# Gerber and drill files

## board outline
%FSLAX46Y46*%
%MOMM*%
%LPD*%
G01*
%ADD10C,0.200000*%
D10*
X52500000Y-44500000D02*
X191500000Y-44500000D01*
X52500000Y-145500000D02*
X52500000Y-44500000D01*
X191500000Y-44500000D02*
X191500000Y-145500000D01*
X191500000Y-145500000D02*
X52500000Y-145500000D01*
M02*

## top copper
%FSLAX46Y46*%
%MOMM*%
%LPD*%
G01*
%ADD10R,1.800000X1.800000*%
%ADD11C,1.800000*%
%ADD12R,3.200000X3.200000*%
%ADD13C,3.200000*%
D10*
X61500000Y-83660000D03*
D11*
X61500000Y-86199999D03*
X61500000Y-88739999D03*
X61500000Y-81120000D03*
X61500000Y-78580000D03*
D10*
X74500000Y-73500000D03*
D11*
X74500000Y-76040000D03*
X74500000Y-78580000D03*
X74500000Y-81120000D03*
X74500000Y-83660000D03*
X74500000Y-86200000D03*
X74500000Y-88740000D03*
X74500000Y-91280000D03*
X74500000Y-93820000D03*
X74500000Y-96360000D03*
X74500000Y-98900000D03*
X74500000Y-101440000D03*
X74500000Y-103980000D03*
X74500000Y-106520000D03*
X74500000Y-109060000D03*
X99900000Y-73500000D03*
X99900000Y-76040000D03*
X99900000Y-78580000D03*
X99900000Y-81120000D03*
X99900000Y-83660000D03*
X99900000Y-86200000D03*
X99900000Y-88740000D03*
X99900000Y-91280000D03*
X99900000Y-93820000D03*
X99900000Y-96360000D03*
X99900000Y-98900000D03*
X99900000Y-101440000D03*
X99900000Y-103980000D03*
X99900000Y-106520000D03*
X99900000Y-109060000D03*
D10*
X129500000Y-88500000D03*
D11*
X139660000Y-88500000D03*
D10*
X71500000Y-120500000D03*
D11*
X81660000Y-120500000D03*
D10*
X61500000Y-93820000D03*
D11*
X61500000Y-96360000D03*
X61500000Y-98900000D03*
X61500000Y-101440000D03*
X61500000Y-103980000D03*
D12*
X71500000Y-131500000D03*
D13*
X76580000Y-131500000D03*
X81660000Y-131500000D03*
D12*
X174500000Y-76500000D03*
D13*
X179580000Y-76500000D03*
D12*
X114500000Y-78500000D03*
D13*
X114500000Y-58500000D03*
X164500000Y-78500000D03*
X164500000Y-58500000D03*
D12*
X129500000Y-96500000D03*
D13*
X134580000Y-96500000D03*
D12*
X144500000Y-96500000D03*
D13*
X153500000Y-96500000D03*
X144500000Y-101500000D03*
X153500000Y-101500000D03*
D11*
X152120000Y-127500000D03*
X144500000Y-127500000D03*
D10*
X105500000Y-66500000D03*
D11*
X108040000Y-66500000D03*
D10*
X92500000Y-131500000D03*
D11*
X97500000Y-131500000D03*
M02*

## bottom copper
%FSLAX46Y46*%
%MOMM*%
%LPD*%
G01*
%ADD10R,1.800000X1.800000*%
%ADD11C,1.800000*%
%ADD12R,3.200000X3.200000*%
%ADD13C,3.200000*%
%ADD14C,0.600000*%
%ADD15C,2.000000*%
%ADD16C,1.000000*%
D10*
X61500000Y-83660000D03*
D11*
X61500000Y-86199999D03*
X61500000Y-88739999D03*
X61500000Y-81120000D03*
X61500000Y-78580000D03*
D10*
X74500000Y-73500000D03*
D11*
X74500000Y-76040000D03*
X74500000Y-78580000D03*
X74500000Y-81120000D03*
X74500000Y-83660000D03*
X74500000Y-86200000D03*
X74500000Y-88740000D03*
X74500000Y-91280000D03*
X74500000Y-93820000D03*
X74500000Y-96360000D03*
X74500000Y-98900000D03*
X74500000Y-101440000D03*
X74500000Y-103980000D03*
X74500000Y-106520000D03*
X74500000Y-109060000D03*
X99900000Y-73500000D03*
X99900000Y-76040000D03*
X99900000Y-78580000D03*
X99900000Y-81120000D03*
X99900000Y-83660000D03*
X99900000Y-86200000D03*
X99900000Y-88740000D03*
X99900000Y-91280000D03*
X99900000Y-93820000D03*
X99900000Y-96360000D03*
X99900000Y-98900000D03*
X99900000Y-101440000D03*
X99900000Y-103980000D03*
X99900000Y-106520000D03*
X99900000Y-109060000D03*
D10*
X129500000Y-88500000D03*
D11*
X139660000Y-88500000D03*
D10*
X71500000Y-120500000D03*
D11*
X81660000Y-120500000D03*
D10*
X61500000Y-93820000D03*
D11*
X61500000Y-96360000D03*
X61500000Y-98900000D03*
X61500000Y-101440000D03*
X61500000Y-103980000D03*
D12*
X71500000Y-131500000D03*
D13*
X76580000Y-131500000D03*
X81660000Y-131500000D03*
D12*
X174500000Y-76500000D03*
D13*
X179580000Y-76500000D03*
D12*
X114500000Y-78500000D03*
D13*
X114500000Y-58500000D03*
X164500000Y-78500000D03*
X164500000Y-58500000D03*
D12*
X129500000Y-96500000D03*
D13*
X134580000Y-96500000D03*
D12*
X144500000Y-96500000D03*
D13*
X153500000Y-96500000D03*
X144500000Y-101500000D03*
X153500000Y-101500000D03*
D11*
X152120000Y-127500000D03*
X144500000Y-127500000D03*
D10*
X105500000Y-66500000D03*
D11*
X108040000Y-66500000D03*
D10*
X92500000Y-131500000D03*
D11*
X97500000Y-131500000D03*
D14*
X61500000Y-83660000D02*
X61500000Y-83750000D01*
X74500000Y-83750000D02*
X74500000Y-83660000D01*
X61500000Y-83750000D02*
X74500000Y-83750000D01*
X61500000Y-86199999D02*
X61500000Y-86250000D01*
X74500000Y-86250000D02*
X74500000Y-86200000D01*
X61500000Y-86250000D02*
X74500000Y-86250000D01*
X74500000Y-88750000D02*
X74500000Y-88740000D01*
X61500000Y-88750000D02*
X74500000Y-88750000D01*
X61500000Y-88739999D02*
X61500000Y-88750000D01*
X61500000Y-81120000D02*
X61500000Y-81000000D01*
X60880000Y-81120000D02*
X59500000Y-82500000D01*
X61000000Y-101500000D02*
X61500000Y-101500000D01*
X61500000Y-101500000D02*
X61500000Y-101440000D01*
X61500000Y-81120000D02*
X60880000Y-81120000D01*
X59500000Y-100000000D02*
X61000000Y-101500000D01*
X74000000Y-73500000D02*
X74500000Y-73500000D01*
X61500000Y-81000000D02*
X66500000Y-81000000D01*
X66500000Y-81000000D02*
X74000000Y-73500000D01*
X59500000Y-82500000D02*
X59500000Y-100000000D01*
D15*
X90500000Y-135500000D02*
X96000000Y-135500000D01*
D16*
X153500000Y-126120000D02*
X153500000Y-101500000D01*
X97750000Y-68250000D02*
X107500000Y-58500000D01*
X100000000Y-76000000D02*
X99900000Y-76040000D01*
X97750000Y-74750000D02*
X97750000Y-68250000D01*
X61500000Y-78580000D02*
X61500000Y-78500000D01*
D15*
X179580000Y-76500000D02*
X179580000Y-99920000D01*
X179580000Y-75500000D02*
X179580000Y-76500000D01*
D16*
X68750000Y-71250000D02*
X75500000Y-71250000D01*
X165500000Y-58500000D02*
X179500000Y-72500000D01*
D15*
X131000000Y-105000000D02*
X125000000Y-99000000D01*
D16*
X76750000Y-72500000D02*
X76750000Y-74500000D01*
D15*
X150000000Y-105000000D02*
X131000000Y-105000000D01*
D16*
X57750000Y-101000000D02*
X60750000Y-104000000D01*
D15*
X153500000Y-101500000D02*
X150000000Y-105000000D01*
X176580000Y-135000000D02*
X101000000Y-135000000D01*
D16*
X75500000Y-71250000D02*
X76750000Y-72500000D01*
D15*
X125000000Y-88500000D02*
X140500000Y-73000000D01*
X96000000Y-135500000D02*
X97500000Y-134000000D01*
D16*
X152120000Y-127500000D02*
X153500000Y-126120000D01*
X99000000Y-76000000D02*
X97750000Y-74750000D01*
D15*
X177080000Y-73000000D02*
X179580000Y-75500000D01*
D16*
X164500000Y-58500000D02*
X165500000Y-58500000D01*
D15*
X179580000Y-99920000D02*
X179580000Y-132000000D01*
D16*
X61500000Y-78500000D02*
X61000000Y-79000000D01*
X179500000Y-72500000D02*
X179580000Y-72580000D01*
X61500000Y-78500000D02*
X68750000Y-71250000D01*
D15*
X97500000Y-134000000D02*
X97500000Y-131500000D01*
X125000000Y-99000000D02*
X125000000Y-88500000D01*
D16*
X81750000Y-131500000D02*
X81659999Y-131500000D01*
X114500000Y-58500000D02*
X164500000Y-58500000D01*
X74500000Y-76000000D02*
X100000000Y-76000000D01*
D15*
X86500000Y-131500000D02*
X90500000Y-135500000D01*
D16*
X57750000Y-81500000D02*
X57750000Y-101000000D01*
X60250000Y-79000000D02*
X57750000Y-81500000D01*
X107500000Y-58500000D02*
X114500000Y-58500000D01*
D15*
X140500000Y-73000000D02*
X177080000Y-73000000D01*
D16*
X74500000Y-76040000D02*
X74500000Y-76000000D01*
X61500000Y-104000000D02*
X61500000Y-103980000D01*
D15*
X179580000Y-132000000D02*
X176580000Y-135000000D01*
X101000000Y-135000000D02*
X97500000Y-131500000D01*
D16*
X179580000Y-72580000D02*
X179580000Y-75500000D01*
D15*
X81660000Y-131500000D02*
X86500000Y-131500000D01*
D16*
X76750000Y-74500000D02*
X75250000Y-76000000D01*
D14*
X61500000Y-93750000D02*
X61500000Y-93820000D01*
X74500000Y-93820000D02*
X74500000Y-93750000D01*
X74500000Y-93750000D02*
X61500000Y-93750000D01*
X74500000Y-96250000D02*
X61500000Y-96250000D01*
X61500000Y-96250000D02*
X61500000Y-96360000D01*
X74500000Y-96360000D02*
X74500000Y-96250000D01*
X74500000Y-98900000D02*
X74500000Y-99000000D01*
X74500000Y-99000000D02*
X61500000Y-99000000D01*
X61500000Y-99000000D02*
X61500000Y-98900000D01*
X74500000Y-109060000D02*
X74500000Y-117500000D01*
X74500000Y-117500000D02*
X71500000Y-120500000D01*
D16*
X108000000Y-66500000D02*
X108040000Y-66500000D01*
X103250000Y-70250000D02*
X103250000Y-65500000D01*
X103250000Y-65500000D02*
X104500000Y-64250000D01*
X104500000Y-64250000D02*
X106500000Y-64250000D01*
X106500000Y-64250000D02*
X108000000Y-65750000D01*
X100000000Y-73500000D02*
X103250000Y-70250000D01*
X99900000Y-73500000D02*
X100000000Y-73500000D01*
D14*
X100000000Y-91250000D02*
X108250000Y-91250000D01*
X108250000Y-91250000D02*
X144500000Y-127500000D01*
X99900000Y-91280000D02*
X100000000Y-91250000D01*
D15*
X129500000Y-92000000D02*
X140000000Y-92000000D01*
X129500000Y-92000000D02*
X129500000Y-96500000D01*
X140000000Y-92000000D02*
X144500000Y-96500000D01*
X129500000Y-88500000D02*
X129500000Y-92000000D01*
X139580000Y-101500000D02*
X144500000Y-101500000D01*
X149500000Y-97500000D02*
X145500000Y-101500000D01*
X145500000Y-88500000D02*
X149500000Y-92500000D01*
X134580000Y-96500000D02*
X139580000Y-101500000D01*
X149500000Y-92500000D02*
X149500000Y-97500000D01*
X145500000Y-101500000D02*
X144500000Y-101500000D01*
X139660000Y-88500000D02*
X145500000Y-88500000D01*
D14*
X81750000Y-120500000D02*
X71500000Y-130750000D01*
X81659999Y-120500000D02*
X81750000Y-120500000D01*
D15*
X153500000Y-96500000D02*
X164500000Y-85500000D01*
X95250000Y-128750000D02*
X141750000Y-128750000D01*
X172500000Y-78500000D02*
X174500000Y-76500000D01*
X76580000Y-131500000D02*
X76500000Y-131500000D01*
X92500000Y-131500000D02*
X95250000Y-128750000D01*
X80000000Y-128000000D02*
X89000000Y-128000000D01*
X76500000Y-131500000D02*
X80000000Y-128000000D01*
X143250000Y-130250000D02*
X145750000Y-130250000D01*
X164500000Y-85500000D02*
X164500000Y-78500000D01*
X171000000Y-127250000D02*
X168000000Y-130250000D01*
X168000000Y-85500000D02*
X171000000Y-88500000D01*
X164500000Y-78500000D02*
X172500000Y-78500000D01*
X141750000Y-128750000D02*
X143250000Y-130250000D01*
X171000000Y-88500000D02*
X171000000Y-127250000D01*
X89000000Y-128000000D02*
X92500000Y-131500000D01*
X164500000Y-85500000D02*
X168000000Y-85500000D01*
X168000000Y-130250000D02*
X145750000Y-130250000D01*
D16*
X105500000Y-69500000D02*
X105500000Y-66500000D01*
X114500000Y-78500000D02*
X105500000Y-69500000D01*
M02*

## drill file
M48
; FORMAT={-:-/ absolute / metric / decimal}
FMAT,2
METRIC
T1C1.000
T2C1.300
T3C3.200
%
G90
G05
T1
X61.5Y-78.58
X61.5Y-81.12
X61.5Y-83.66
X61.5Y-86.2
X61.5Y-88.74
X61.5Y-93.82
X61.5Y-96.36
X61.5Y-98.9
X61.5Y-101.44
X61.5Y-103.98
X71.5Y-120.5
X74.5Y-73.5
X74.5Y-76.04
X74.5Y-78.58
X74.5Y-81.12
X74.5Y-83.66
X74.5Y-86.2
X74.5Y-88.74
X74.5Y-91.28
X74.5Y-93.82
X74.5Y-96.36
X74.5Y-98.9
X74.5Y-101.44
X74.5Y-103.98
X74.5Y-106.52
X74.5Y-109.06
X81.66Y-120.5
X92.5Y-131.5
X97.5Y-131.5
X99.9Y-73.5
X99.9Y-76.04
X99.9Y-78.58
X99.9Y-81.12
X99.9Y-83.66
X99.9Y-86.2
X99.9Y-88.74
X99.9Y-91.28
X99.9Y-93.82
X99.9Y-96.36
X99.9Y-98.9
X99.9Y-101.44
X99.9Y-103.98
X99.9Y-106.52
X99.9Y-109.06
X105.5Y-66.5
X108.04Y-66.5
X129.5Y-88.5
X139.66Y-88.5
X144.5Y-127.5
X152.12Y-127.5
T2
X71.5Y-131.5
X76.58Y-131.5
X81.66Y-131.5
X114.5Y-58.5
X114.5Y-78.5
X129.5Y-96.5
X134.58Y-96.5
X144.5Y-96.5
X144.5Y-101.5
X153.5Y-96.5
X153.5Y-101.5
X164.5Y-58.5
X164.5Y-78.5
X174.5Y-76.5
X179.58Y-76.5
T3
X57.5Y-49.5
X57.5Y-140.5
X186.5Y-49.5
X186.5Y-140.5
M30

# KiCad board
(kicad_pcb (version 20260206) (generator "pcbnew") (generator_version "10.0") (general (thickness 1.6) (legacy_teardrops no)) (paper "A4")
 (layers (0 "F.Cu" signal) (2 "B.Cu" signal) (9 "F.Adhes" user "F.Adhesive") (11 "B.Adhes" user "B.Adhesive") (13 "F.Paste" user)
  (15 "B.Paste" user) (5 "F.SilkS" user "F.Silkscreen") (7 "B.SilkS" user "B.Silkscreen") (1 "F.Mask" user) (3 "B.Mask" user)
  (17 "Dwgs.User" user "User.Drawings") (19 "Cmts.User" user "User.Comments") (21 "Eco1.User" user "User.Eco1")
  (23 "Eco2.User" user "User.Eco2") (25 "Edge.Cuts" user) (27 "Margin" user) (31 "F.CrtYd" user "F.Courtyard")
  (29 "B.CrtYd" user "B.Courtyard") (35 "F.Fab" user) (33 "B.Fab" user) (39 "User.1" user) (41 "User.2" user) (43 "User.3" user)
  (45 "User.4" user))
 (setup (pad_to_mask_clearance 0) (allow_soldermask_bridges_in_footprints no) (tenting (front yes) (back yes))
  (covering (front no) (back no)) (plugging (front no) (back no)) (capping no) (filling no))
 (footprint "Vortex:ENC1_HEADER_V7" (layer "F.Cu") (at 61.5 83.5 -90)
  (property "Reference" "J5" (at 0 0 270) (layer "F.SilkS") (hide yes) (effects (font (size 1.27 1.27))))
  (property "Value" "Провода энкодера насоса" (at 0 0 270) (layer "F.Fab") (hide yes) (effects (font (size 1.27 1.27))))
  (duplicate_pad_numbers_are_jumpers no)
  (pad "1" thru_hole rect (at 0.16 0 270) (size 1.8 1.8) (drill 1) (layers "*.Cu") (remove_unused_layers no) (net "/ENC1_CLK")
   (thermal_bridge_angle 45))
  (pad "2" thru_hole circle (at 2.699999 0 270) (size 1.8 1.8) (drill 1) (layers "*.Cu") (remove_unused_layers no) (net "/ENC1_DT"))
  (pad "3" thru_hole circle (at 5.239999 0 270) (size 1.8 1.8) (drill 1) (layers "*.Cu") (remove_unused_layers no) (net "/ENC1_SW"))
  (pad "4" thru_hole circle (at -2.38 0 270) (size 1.8 1.8) (drill 1) (layers "*.Cu") (remove_unused_layers no) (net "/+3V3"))
  (pad "5" thru_hole circle (at -4.92 0 270) (size 1.8 1.8) (drill 1) (layers "*.Cu") (remove_unused_layers no) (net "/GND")))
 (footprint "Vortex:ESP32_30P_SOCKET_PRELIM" (layer "F.Cu") (at 74.5 73.5)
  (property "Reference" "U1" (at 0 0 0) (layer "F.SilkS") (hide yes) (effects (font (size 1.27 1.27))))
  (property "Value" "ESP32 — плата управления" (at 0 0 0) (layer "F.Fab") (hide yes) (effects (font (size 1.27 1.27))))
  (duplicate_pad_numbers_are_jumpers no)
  (pad "1" thru_hole rect (at 0 0) (size 1.8 1.8) (drill 1) (layers "*.Cu") (remove_unused_layers no) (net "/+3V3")
   (thermal_bridge_angle 45))
  (pad "2" thru_hole circle (at 0 2.54) (size 1.8 1.8) (drill 1) (layers "*.Cu") (remove_unused_layers no) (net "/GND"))
  (pad "3" thru_hole circle (at 0 5.08) (size 1.8 1.8) (drill 1) (layers "*.Cu") (remove_unused_layers no) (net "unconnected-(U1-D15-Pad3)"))
  (pad "4" thru_hole circle (at 0 7.62) (size 1.8 1.8) (drill 1) (layers "*.Cu") (remove_unused_layers no) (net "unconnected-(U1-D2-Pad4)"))
  (pad "5" thru_hole circle (at 0 10.16) (size 1.8 1.8) (drill 1) (layers "*.Cu") (remove_unused_layers no) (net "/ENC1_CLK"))
  (pad "6" thru_hole circle (at 0 12.7) (size 1.8 1.8) (drill 1) (layers "*.Cu") (remove_unused_layers no) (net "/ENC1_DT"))
  (pad "7" thru_hole circle (at 0 15.24) (size 1.8 1.8) (drill 1) (layers "*.Cu") (remove_unused_layers no) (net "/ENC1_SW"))
  (pad "8" thru_hole circle (at 0 17.78) (size 1.8 1.8) (drill 1) (layers "*.Cu") (remove_unused_layers no) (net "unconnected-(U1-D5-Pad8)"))
  (pad "9" thru_hole circle (at 0 20.32) (size 1.8 1.8) (drill 1) (layers "*.Cu") (remove_unused_layers no) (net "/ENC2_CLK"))
  (pad "10" thru_hole circle (at 0 22.86) (size 1.8 1.8) (drill 1) (layers "*.Cu") (remove_unused_layers no) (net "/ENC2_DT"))
  (pad "11" thru_hole circle (at 0 25.4) (size 1.8 1.8) (drill 1) (layers "*.Cu") (remove_unused_layers no) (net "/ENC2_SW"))
  (pad "12" thru_hole circle (at 0 27.94) (size 1.8 1.8) (drill 1) (layers "*.Cu") (remove_unused_layers no)
   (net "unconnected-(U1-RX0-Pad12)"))
  (pad "13" thru_hole circle (at 0 30.48) (size 1.8 1.8) (drill 1) (layers "*.Cu") (remove_unused_layers no)
   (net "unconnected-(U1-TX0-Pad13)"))
  (pad "14" thru_hole circle (at 0 33.02) (size 1.8 1.8) (drill 1) (layers "*.Cu") (remove_unused_layers no)
   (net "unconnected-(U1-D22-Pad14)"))
  (pad "15" thru_hole circle (at 0 35.56) (size 1.8 1.8) (drill 1) (layers "*.Cu") (remove_unused_layers no) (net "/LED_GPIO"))
  (pad "16" thru_hole circle (at 25.4 0) (size 1.8 1.8) (drill 1) (layers "*.Cu") (remove_unused_layers no) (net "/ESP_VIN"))
  (pad "17" thru_hole circle (at 25.4 2.54) (size 1.8 1.8) (drill 1) (layers "*.Cu") (remove_unused_layers no) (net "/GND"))
  (pad "18" thru_hole circle (at 25.4 5.08) (size 1.8 1.8) (drill 1) (layers "*.Cu") (remove_unused_layers no)
   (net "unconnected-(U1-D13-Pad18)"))
  (pad "19" thru_hole circle (at 25.4 7.62) (size 1.8 1.8) (drill 1) (layers "*.Cu") (remove_unused_layers no)
   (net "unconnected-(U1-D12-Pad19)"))
  (pad "20" thru_hole circle (at 25.4 10.16) (size 1.8 1.8) (drill 1) (layers "*.Cu") (remove_unused_layers no)
   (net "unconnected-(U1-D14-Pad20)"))
  (pad "21" thru_hole circle (at 25.4 12.7) (size 1.8 1.8) (drill 1) (layers "*.Cu") (remove_unused_layers no)
   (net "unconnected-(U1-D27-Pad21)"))
  (pad "22" thru_hole circle (at 25.4 15.24) (size 1.8 1.8) (drill 1) (layers "*.Cu") (remove_unused_layers no)
   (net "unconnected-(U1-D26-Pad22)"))
  (pad "23" thru_hole circle (at 25.4 17.78) (size 1.8 1.8) (drill 1) (layers "*.Cu") (remove_unused_layers no) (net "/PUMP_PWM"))
  (pad "24" thru_hole circle (at 25.4 20.32) (size 1.8 1.8) (drill 1) (layers "*.Cu") (remove_unused_layers no)
   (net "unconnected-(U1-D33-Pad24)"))
  (pad "25" thru_hole circle (at 25.4 22.86) (size 1.8 1.8) (drill 1) (layers "*.Cu") (remove_unused_layers no)
   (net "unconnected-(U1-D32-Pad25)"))
  (pad "26" thru_hole circle (at 25.4 25.4) (size 1.8 1.8) (drill 1) (layers "*.Cu") (remove_unused_layers no)
   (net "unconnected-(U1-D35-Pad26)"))
  (pad "27" thru_hole circle (at 25.4 27.94) (size 1.8 1.8) (drill 1) (layers "*.Cu") (remove_unused_layers no)
   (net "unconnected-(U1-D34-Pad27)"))
  (pad "28" thru_hole circle (at 25.4 30.48) (size 1.8 1.8) (drill 1) (layers "*.Cu") (remove_unused_layers no)
   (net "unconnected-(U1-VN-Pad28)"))
  (pad "29" thru_hole circle (at 25.4 33.02) (size 1.8 1.8) (drill 1) (layers "*.Cu") (remove_unused_layers no)
   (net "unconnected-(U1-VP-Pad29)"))
  (pad "30" thru_hole circle (at 25.4 35.56) (size 1.8 1.8) (drill 1) (layers "*.Cu") (remove_unused_layers no)
   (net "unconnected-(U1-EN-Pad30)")))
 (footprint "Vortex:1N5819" (layer "F.Cu") (at 129.5 88.5)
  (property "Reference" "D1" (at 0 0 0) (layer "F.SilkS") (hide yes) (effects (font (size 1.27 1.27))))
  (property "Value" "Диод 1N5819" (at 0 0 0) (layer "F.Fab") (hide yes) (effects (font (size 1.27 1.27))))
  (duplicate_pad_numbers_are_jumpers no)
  (pad "1" thru_hole rect (at 0 0) (size 1.8 1.8) (drill 1) (layers "*.Cu") (remove_unused_layers no) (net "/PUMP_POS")
   (thermal_bridge_angle 45))
  (pad "2" thru_hole circle (at 10.16 0) (size 1.8 1.8) (drill 1) (layers "*.Cu") (remove_unused_layers no) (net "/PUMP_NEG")))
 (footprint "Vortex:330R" (layer "F.Cu") (at 71.5 120.5)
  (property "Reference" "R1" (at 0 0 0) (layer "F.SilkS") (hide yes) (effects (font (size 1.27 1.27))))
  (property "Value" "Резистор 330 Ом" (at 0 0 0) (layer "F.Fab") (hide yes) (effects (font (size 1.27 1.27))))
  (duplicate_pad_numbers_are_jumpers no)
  (pad "1" thru_hole rect (at 0 0) (size 1.8 1.8) (drill 1) (layers "*.Cu") (remove_unused_layers no) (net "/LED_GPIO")
   (thermal_bridge_angle 45))
  (pad "2" thru_hole circle (at 10.16 0) (size 1.8 1.8) (drill 1) (layers "*.Cu") (remove_unused_layers no) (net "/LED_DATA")))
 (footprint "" (layer "F.Cu") (at 57.5 140.5)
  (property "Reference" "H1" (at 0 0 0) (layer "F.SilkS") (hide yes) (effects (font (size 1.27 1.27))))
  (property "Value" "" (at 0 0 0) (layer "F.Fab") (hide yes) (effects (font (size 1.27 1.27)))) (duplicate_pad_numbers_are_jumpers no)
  (pad "" np_thru_hole circle (at 0 0) (size 3.2 3.2) (drill 3.2) (layers "*.Cu")))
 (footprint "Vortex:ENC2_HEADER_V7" (layer "F.Cu") (at 61.5 96.5 -90)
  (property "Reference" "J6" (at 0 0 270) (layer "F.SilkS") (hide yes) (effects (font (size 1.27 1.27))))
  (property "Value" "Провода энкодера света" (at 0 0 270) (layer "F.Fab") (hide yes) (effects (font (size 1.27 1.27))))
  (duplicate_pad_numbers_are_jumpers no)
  (pad "1" thru_hole rect (at -2.68 0 270) (size 1.8 1.8) (drill 1) (layers "*.Cu") (remove_unused_layers no) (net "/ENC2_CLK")
   (thermal_bridge_angle 45))
  (pad "2" thru_hole circle (at -0.14 0 270) (size 1.8 1.8) (drill 1) (layers "*.Cu") (remove_unused_layers no) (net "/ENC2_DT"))
  (pad "3" thru_hole circle (at 2.4 0 270) (size 1.8 1.8) (drill 1) (layers "*.Cu") (remove_unused_layers no) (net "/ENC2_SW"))
  (pad "4" thru_hole circle (at 4.94 0 270) (size 1.8 1.8) (drill 1) (layers "*.Cu") (remove_unused_layers no) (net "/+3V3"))
  (pad "5" thru_hole circle (at 7.48 0 270) (size 1.8 1.8) (drill 1) (layers "*.Cu") (remove_unused_layers no) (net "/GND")))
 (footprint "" (layer "F.Cu") (at 57.5 49.5)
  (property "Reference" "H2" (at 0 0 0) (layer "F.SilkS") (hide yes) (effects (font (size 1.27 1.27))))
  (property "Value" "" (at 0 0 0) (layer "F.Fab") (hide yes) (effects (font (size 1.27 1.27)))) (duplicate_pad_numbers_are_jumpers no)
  (pad "" np_thru_hole circle (at 0 0) (size 3.2 3.2) (drill 3.2) (layers "*.Cu")))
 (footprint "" (layer "F.Cu") (at 186.5 140.5)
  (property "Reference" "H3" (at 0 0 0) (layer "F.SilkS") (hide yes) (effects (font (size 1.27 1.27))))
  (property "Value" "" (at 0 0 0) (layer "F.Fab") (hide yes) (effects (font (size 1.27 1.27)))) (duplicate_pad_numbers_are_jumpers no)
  (pad "" np_thru_hole circle (at 0 0) (size 3.2 3.2) (drill 3.2) (layers "*.Cu")))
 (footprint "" (layer "F.Cu") (at 186.5 49.5)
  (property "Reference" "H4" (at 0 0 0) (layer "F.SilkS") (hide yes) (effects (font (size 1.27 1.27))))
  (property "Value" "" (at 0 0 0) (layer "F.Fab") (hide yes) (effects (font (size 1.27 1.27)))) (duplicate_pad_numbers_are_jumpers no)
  (pad "" np_thru_hole circle (at 0 0) (size 3.2 3.2) (drill 3.2) (layers "*.Cu")))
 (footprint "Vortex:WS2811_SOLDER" (layer "F.Cu") (at 71.5 131.5)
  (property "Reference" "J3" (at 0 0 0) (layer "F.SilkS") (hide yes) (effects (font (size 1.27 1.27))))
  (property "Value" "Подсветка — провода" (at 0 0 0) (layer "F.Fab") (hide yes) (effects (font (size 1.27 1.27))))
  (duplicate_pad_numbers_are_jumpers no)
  (pad "1" thru_hole rect (at 0 0) (size 3.2 3.2) (drill 1.3) (layers "*.Cu") (remove_unused_layers no) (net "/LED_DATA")
   (thermal_bridge_angle 45))
  (pad "2" thru_hole circle (at 5.08 0) (size 3.2 3.2) (drill 1.3) (layers "*.Cu") (remove_unused_layers no) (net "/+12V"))
  (pad "3" thru_hole circle (at 10.16 0) (size 3.2 3.2) (drill 1.3) (layers "*.Cu") (remove_unused_layers no) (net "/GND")))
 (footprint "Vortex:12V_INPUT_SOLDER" (layer "F.Cu") (at 174.5 76.5)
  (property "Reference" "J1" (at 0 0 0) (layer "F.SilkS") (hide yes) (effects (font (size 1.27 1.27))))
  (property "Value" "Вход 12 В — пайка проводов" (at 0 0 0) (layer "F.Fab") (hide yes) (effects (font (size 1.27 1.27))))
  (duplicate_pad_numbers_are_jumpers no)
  (pad "1" thru_hole rect (at 0 0) (size 3.2 3.2) (drill 1.3) (layers "*.Cu") (remove_unused_layers no) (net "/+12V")
   (thermal_bridge_angle 45))
  (pad "2" thru_hole circle (at 5.08 0) (size 3.2 3.2) (drill 1.3) (layers "*.Cu") (remove_unused_layers no) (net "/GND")))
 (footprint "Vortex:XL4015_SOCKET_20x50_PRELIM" (layer "F.Cu") (at 114.5 78.5 90)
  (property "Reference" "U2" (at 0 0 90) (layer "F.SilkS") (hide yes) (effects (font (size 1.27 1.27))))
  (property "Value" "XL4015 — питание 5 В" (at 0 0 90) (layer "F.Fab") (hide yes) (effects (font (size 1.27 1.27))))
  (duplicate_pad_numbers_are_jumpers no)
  (pad "1" thru_hole rect (at 0 0 90) (size 3.2 3.2) (drill 1.3) (layers "*.Cu") (remove_unused_layers no) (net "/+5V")
   (thermal_bridge_angle 45))
  (pad "2" thru_hole circle (at 20 0 90) (size 3.2 3.2) (drill 1.3) (layers "*.Cu") (remove_unused_layers no) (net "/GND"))
  (pad "3" thru_hole circle (at 0 50 90) (size 3.2 3.2) (drill 1.3) (layers "*.Cu") (remove_unused_layers no) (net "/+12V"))
  (pad "4" thru_hole circle (at 20 50 90) (size 3.2 3.2) (drill 1.3) (layers "*.Cu") (remove_unused_layers no) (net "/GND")))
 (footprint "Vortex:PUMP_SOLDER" (layer "F.Cu") (at 129.5 96.5)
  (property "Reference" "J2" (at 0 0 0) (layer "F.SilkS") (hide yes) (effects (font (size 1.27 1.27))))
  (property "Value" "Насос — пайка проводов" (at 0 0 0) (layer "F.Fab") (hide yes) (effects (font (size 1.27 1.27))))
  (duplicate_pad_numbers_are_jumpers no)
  (pad "1" thru_hole rect (at 0 0) (size 3.2 3.2) (drill 1.3) (layers "*.Cu") (remove_unused_layers no) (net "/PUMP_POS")
   (thermal_bridge_angle 45))
  (pad "2" thru_hole circle (at 5.08 0) (size 3.2 3.2) (drill 1.3) (layers "*.Cu") (remove_unused_layers no) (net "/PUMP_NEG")))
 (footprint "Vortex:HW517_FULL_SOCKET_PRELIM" (layer "F.Cu") (at 144.5 96.5)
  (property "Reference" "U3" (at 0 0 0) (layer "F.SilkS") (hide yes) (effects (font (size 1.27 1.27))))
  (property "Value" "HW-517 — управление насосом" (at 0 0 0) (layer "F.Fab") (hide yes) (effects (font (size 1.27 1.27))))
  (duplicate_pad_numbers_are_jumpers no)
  (pad "1" thru_hole rect (at 0 0) (size 3.2 3.2) (drill 1.3) (layers "*.Cu") (remove_unused_layers no) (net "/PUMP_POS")
   (thermal_bridge_angle 45))
  (pad "2" thru_hole circle (at 9 0) (size 3.2 3.2) (drill 1.3) (layers "*.Cu") (remove_unused_layers no) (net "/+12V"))
  (pad "3" thru_hole circle (at 0 5) (size 3.2 3.2) (drill 1.3) (layers "*.Cu") (remove_unused_layers no) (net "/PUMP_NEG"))
  (pad "4" thru_hole circle (at 9 5) (size 3.2 3.2) (drill 1.3) (layers "*.Cu") (remove_unused_layers no) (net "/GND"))
  (pad "5" thru_hole circle (at 7.62 31) (size 1.8 1.8) (drill 1) (layers "*.Cu") (remove_unused_layers no) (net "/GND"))
  (pad "6" thru_hole circle (at 0 31) (size 1.8 1.8) (drill 1) (layers "*.Cu") (remove_unused_layers no) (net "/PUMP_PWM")))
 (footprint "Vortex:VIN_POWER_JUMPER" (layer "F.Cu") (at 105.5 66.5)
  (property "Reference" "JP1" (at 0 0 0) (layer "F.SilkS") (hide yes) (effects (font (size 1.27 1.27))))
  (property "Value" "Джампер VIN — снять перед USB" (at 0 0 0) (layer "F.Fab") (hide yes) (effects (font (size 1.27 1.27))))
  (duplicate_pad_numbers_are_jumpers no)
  (pad "1" thru_hole rect (at 0 0) (size 1.8 1.8) (drill 1) (layers "*.Cu") (remove_unused_layers no) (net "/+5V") (thermal_bridge_angle 45))
  (pad "2" thru_hole circle (at 2.54 0) (size 1.8 1.8) (drill 1) (layers "*.Cu") (remove_unused_layers no) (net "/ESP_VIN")))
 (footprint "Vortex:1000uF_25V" (layer "F.Cu") (at 92.5 131.5)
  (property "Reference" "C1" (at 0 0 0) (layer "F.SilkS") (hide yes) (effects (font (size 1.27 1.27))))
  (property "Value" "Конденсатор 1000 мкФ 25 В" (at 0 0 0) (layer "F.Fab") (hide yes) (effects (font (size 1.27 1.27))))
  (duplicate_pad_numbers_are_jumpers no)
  (pad "1" thru_hole rect (at 0 0) (size 1.8 1.8) (drill 1) (layers "*.Cu") (remove_unused_layers no) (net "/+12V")
   (thermal_bridge_angle 45))
  (pad "2" thru_hole circle (at 5 0) (size 1.8 1.8) (drill 1) (layers "*.Cu") (remove_unused_layers no) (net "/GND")))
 (gr_line (start 52.5 44.5) (end 191.5 44.5) (stroke (width 0.2) (type default)) (layer "Edge.Cuts"))
 (gr_line (start 52.5 145.5) (end 52.5 44.5) (stroke (width 0.2) (type default)) (layer "Edge.Cuts"))
 (gr_line (start 191.5 44.5) (end 191.5 145.5) (stroke (width 0.2) (type default)) (layer "Edge.Cuts"))
 (gr_line (start 191.5 145.5) (end 52.5 145.5) (stroke (width 0.2) (type default)) (layer "Edge.Cuts"))
 (segment (start 61.5 83.66) (end 61.5 83.75) (width 0.6) (layer "B.Cu") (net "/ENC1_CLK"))
 (segment (start 74.5 83.75) (end 74.5 83.66) (width 0.6) (layer "B.Cu") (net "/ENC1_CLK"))
 (segment (start 61.5 83.75) (end 74.5 83.75) (width 0.6) (layer "B.Cu") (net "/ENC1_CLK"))
 (segment (start 61.5 86.199999) (end 61.5 86.25) (width 0.6) (layer "B.Cu") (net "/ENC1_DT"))
 (segment (start 74.5 86.25) (end 74.5 86.2) (width 0.6) (layer "B.Cu") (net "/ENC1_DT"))
 (segment (start 61.5 86.25) (end 74.5 86.25) (width 0.6) (layer "B.Cu") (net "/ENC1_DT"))
 (segment (start 74.5 88.75) (end 74.5 88.74) (width 0.6) (layer "B.Cu") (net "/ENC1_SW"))
 (segment (start 61.5 88.75) (end 74.5 88.75) (width 0.6) (layer "B.Cu") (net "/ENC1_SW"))
 (segment (start 61.5 88.739999) (end 61.5 88.75) (width 0.6) (layer "B.Cu") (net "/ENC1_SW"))
 (segment (start 61.5 81.12) (end 61.5 81) (width 0.6) (layer "B.Cu") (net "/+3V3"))
 (segment (start 60.88 81.12) (end 59.5 82.5) (width 0.6) (layer "B.Cu") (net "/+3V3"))
 (segment (start 61 101.5) (end 61.5 101.5) (width 0.6) (layer "B.Cu") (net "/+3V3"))
 (segment (start 61.5 101.5) (end 61.5 101.44) (width 0.6) (layer "B.Cu") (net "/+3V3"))
 (segment (start 61.5 81.12) (end 60.88 81.12) (width 0.6) (layer "B.Cu") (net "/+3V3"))
 (segment (start 59.5 100) (end 61 101.5) (width 0.6) (layer "B.Cu") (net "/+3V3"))
 (segment (start 74 73.5) (end 74.5 73.5) (width 0.6) (layer "B.Cu") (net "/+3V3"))
 (segment (start 61.5 81) (end 66.5 81) (width 0.6) (layer "B.Cu") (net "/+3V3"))
 (segment (start 66.5 81) (end 74 73.5) (width 0.6) (layer "B.Cu") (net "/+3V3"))
 (segment (start 59.5 82.5) (end 59.5 100) (width 0.6) (layer "B.Cu") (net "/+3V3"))
 (segment (start 90.5 135.5) (end 96 135.5) (width 2) (layer "B.Cu") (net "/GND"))
 (segment (start 153.5 126.12) (end 153.5 101.5) (width 1) (layer "B.Cu") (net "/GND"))
 (segment (start 97.75 68.25) (end 107.5 58.5) (width 1) (layer "B.Cu") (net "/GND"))
 (segment (start 100 76) (end 99.9 76.04) (width 1) (layer "B.Cu") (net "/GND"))
 (segment (start 97.75 74.75) (end 97.75 68.25) (width 1) (layer "B.Cu") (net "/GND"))
 (segment (start 61.5 78.58) (end 61.5 78.5) (width 1) (layer "B.Cu") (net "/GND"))
 (segment (start 179.58 76.5) (end 179.58 99.92) (width 2) (layer "B.Cu") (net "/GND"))
 (segment (start 179.58 75.5) (end 179.58 76.5) (width 2) (layer "B.Cu") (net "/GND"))
 (segment (start 68.75 71.25) (end 75.5 71.25) (width 1) (layer "B.Cu") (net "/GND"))
 (segment (start 165.5 58.5) (end 179.5 72.5) (width 1) (layer "B.Cu") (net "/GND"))
 (segment (start 131 105) (end 125 99) (width 2) (layer "B.Cu") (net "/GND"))
 (segment (start 76.75 72.5) (end 76.75 74.5) (width 1) (layer "B.Cu") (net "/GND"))
 (segment (start 150 105) (end 131 105) (width 2) (layer "B.Cu") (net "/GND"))
 (segment (start 57.75 101) (end 60.75 104) (width 1) (layer "B.Cu") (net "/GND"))
 (segment (start 153.5 101.5) (end 150 105) (width 2) (layer "B.Cu") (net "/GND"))
 (segment (start 176.58 135) (end 101 135) (width 2) (layer "B.Cu") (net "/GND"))
 (segment (start 75.5 71.25) (end 76.75 72.5) (width 1) (layer "B.Cu") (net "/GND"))
 (segment (start 125 88.5) (end 140.5 73) (width 2) (layer "B.Cu") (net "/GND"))
 (segment (start 96 135.5) (end 97.5 134) (width 2) (layer "B.Cu") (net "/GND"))
 (segment (start 152.12 127.5) (end 153.5 126.12) (width 1) (layer "B.Cu") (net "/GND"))
 (segment (start 99 76) (end 97.75 74.75) (width 1) (layer "B.Cu") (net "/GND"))
 (segment (start 177.08 73) (end 179.58 75.5) (width 2) (layer "B.Cu") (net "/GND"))
 (segment (start 164.5 58.5) (end 165.5 58.5) (width 1) (layer "B.Cu") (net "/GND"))
 (segment (start 179.58 99.92) (end 179.58 132) (width 2) (layer "B.Cu") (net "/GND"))
 (segment (start 61.5 78.5) (end 61 79) (width 1) (layer "B.Cu") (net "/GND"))
 (segment (start 179.5 72.5) (end 179.58 72.58) (width 1) (layer "B.Cu") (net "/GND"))
 (segment (start 61.5 78.5) (end 68.75 71.25) (width 1) (layer "B.Cu") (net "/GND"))
 (segment (start 97.5 134) (end 97.5 131.5) (width 2) (layer "B.Cu") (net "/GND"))
 (segment (start 125 99) (end 125 88.5) (width 2) (layer "B.Cu") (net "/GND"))
 (segment (start 81.75 131.5) (end 81.659999 131.5) (width 1) (layer "B.Cu") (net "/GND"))
 (segment (start 114.5 58.5) (end 164.5 58.5) (width 1) (layer "B.Cu") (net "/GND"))
 (segment (start 74.5 76) (end 100 76) (width 1) (layer "B.Cu") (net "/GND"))
 (segment (start 86.5 131.5) (end 90.5 135.5) (width 2) (layer "B.Cu") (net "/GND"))
 (segment (start 57.75 81.5) (end 57.75 101) (width 1) (layer "B.Cu") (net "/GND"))
 (segment (start 60.25 79) (end 57.75 81.5) (width 1) (layer "B.Cu") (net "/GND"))
 (segment (start 107.5 58.5) (end 114.5 58.5) (width 1) (layer "B.Cu") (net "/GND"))
 (segment (start 140.5 73) (end 177.08 73) (width 2) (layer "B.Cu") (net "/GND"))
 (segment (start 74.5 76.04) (end 74.5 76) (width 1) (layer "B.Cu") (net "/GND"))
 (segment (start 61.5 104) (end 61.5 103.98) (width 1) (layer "B.Cu") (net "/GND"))
 (segment (start 179.58 132) (end 176.58 135) (width 2) (layer "B.Cu") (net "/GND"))
 (segment (start 101 135) (end 97.5 131.5) (width 2) (layer "B.Cu") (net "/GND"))
 (segment (start 179.58 72.58) (end 179.58 75.5) (width 1) (layer "B.Cu") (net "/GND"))
 (segment (start 81.66 131.5) (end 86.5 131.5) (width 2) (layer "B.Cu") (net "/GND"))
 (segment (start 76.75 74.5) (end 75.25 76) (width 1) (layer "B.Cu") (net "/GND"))
 (segment (start 61.5 93.75) (end 61.5 93.82) (width 0.6) (layer "B.Cu") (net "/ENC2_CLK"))
 (segment (start 74.5 93.82) (end 74.5 93.75) (width 0.6) (layer "B.Cu") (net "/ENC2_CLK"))
 (segment (start 74.5 93.75) (end 61.5 93.75) (width 0.6) (layer "B.Cu") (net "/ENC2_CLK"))
 (segment (start 74.5 96.25) (end 61.5 96.25) (width 0.6) (layer "B.Cu") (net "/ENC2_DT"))
 (segment (start 61.5 96.25) (end 61.5 96.36) (width 0.6) (layer "B.Cu") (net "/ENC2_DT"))
 (segment (start 74.5 96.36) (end 74.5 96.25) (width 0.6) (layer "B.Cu") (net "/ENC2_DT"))
 (segment (start 74.5 98.9) (end 74.5 99) (width 0.6) (layer "B.Cu") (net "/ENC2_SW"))
 (segment (start 74.5 99) (end 61.5 99) (width 0.6) (layer "B.Cu") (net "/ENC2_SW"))
 (segment (start 61.5 99) (end 61.5 98.9) (width 0.6) (layer "B.Cu") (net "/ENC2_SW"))
 (segment (start 74.5 109.06) (end 74.5 117.5) (width 0.6) (layer "B.Cu") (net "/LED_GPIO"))
 (segment (start 74.5 117.5) (end 71.5 120.5) (width 0.6) (layer "B.Cu") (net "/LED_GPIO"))
 (segment (start 108 66.5) (end 108.04 66.5) (width 1) (layer "B.Cu") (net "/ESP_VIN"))
 (segment (start 103.25 70.25) (end 103.25 65.5) (width 1) (layer "B.Cu") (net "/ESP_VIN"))
 (segment (start 103.25 65.5) (end 104.5 64.25) (width 1) (layer "B.Cu") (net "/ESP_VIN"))
 (segment (start 104.5 64.25) (end 106.5 64.25) (width 1) (layer "B.Cu") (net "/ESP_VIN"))
 (segment (start 106.5 64.25) (end 108 65.75) (width 1) (layer "B.Cu") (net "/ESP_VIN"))
 (segment (start 100 73.5) (end 103.25 70.25) (width 1) (layer "B.Cu") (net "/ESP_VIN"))
 (segment (start 99.9 73.5) (end 100 73.5) (width 1) (layer "B.Cu") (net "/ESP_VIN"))
 (segment (start 100 91.25) (end 108.25 91.25) (width 0.6) (layer "B.Cu") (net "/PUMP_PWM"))
 (segment (start 108.25 91.25) (end 144.5 127.5) (width 0.6) (layer "B.Cu") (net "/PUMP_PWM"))
 (segment (start 99.9 91.28) (end 100 91.25) (width 0.6) (layer "B.Cu") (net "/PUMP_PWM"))
 (segment (start 129.5 92) (end 140 92) (width 2) (layer "B.Cu") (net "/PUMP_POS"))
 (segment (start 129.5 92) (end 129.5 96.5) (width 2) (layer "B.Cu") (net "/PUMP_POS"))
 (segment (start 140 92) (end 144.5 96.5) (width 2) (layer "B.Cu") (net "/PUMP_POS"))
 (segment (start 129.5 88.5) (end 129.5 92) (width 2) (layer "B.Cu") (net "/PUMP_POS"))
 (segment (start 139.58 101.5) (end 144.5 101.5) (width 2) (layer "B.Cu") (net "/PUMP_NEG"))
 (segment (start 149.5 97.5) (end 145.5 101.5) (width 2) (layer "B.Cu") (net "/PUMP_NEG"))
 (segment (start 145.5 88.5) (end 149.5 92.5) (width 2) (layer "B.Cu") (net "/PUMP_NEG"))
 (segment (start 134.58 96.5) (end 139.58 101.5) (width 2) (layer "B.Cu") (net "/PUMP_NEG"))
 (segment (start 149.5 92.5) (end 149.5 97.5) (width 2) (layer "B.Cu") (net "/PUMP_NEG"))
 (segment (start 145.5 101.5) (end 144.5 101.5) (width 2) (layer "B.Cu") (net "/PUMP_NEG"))
 (segment (start 139.66 88.5) (end 145.5 88.5) (width 2) (layer "B.Cu") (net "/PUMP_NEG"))
 (segment (start 81.75 120.5) (end 71.5 130.75) (width 0.6) (layer "B.Cu") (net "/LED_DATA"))
 (segment (start 81.659999 120.5) (end 81.75 120.5) (width 0.6) (layer "B.Cu") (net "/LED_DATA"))
 (segment (start 153.5 96.5) (end 164.5 85.5) (width 2) (layer "B.Cu") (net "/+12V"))
 (segment (start 95.25 128.75) (end 141.75 128.75) (width 2) (layer "B.Cu") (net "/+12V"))
 (segment (start 172.5 78.5) (end 174.5 76.5) (width 2) (layer "B.Cu") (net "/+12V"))
 (segment (start 76.58 131.5) (end 76.5 131.5) (width 2) (layer "B.Cu") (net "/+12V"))
 (segment (start 92.5 131.5) (end 95.25 128.75) (width 2) (layer "B.Cu") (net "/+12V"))
 (segment (start 80 128) (end 89 128) (width 2) (layer "B.Cu") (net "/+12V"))
 (segment (start 76.5 131.5) (end 80 128) (width 2) (layer "B.Cu") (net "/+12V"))
 (segment (start 143.25 130.25) (end 145.75 130.25) (width 2) (layer "B.Cu") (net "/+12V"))
 (segment (start 164.5 85.5) (end 164.5 78.5) (width 2) (layer "B.Cu") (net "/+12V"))
 (segment (start 171 127.25) (end 168 130.25) (width 2) (layer "B.Cu") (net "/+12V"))
 (segment (start 168 85.5) (end 171 88.5) (width 2) (layer "B.Cu") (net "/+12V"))
 (segment (start 164.5 78.5) (end 172.5 78.5) (width 2) (layer "B.Cu") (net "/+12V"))
 (segment (start 141.75 128.75) (end 143.25 130.25) (width 2) (layer "B.Cu") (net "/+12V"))
 (segment (start 171 88.5) (end 171 127.25) (width 2) (layer "B.Cu") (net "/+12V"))
 (segment (start 89 128) (end 92.5 131.5) (width 2) (layer "B.Cu") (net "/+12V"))
 (segment (start 164.5 85.5) (end 168 85.5) (width 2) (layer "B.Cu") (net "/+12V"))
 (segment (start 168 130.25) (end 145.75 130.25) (width 2) (layer "B.Cu") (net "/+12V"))
 (segment (start 105.5 69.5) (end 105.5 66.5) (width 1) (layer "B.Cu") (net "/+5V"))
 (segment (start 114.5 78.5) (end 105.5 69.5) (width 1) (layer "B.Cu") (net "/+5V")))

